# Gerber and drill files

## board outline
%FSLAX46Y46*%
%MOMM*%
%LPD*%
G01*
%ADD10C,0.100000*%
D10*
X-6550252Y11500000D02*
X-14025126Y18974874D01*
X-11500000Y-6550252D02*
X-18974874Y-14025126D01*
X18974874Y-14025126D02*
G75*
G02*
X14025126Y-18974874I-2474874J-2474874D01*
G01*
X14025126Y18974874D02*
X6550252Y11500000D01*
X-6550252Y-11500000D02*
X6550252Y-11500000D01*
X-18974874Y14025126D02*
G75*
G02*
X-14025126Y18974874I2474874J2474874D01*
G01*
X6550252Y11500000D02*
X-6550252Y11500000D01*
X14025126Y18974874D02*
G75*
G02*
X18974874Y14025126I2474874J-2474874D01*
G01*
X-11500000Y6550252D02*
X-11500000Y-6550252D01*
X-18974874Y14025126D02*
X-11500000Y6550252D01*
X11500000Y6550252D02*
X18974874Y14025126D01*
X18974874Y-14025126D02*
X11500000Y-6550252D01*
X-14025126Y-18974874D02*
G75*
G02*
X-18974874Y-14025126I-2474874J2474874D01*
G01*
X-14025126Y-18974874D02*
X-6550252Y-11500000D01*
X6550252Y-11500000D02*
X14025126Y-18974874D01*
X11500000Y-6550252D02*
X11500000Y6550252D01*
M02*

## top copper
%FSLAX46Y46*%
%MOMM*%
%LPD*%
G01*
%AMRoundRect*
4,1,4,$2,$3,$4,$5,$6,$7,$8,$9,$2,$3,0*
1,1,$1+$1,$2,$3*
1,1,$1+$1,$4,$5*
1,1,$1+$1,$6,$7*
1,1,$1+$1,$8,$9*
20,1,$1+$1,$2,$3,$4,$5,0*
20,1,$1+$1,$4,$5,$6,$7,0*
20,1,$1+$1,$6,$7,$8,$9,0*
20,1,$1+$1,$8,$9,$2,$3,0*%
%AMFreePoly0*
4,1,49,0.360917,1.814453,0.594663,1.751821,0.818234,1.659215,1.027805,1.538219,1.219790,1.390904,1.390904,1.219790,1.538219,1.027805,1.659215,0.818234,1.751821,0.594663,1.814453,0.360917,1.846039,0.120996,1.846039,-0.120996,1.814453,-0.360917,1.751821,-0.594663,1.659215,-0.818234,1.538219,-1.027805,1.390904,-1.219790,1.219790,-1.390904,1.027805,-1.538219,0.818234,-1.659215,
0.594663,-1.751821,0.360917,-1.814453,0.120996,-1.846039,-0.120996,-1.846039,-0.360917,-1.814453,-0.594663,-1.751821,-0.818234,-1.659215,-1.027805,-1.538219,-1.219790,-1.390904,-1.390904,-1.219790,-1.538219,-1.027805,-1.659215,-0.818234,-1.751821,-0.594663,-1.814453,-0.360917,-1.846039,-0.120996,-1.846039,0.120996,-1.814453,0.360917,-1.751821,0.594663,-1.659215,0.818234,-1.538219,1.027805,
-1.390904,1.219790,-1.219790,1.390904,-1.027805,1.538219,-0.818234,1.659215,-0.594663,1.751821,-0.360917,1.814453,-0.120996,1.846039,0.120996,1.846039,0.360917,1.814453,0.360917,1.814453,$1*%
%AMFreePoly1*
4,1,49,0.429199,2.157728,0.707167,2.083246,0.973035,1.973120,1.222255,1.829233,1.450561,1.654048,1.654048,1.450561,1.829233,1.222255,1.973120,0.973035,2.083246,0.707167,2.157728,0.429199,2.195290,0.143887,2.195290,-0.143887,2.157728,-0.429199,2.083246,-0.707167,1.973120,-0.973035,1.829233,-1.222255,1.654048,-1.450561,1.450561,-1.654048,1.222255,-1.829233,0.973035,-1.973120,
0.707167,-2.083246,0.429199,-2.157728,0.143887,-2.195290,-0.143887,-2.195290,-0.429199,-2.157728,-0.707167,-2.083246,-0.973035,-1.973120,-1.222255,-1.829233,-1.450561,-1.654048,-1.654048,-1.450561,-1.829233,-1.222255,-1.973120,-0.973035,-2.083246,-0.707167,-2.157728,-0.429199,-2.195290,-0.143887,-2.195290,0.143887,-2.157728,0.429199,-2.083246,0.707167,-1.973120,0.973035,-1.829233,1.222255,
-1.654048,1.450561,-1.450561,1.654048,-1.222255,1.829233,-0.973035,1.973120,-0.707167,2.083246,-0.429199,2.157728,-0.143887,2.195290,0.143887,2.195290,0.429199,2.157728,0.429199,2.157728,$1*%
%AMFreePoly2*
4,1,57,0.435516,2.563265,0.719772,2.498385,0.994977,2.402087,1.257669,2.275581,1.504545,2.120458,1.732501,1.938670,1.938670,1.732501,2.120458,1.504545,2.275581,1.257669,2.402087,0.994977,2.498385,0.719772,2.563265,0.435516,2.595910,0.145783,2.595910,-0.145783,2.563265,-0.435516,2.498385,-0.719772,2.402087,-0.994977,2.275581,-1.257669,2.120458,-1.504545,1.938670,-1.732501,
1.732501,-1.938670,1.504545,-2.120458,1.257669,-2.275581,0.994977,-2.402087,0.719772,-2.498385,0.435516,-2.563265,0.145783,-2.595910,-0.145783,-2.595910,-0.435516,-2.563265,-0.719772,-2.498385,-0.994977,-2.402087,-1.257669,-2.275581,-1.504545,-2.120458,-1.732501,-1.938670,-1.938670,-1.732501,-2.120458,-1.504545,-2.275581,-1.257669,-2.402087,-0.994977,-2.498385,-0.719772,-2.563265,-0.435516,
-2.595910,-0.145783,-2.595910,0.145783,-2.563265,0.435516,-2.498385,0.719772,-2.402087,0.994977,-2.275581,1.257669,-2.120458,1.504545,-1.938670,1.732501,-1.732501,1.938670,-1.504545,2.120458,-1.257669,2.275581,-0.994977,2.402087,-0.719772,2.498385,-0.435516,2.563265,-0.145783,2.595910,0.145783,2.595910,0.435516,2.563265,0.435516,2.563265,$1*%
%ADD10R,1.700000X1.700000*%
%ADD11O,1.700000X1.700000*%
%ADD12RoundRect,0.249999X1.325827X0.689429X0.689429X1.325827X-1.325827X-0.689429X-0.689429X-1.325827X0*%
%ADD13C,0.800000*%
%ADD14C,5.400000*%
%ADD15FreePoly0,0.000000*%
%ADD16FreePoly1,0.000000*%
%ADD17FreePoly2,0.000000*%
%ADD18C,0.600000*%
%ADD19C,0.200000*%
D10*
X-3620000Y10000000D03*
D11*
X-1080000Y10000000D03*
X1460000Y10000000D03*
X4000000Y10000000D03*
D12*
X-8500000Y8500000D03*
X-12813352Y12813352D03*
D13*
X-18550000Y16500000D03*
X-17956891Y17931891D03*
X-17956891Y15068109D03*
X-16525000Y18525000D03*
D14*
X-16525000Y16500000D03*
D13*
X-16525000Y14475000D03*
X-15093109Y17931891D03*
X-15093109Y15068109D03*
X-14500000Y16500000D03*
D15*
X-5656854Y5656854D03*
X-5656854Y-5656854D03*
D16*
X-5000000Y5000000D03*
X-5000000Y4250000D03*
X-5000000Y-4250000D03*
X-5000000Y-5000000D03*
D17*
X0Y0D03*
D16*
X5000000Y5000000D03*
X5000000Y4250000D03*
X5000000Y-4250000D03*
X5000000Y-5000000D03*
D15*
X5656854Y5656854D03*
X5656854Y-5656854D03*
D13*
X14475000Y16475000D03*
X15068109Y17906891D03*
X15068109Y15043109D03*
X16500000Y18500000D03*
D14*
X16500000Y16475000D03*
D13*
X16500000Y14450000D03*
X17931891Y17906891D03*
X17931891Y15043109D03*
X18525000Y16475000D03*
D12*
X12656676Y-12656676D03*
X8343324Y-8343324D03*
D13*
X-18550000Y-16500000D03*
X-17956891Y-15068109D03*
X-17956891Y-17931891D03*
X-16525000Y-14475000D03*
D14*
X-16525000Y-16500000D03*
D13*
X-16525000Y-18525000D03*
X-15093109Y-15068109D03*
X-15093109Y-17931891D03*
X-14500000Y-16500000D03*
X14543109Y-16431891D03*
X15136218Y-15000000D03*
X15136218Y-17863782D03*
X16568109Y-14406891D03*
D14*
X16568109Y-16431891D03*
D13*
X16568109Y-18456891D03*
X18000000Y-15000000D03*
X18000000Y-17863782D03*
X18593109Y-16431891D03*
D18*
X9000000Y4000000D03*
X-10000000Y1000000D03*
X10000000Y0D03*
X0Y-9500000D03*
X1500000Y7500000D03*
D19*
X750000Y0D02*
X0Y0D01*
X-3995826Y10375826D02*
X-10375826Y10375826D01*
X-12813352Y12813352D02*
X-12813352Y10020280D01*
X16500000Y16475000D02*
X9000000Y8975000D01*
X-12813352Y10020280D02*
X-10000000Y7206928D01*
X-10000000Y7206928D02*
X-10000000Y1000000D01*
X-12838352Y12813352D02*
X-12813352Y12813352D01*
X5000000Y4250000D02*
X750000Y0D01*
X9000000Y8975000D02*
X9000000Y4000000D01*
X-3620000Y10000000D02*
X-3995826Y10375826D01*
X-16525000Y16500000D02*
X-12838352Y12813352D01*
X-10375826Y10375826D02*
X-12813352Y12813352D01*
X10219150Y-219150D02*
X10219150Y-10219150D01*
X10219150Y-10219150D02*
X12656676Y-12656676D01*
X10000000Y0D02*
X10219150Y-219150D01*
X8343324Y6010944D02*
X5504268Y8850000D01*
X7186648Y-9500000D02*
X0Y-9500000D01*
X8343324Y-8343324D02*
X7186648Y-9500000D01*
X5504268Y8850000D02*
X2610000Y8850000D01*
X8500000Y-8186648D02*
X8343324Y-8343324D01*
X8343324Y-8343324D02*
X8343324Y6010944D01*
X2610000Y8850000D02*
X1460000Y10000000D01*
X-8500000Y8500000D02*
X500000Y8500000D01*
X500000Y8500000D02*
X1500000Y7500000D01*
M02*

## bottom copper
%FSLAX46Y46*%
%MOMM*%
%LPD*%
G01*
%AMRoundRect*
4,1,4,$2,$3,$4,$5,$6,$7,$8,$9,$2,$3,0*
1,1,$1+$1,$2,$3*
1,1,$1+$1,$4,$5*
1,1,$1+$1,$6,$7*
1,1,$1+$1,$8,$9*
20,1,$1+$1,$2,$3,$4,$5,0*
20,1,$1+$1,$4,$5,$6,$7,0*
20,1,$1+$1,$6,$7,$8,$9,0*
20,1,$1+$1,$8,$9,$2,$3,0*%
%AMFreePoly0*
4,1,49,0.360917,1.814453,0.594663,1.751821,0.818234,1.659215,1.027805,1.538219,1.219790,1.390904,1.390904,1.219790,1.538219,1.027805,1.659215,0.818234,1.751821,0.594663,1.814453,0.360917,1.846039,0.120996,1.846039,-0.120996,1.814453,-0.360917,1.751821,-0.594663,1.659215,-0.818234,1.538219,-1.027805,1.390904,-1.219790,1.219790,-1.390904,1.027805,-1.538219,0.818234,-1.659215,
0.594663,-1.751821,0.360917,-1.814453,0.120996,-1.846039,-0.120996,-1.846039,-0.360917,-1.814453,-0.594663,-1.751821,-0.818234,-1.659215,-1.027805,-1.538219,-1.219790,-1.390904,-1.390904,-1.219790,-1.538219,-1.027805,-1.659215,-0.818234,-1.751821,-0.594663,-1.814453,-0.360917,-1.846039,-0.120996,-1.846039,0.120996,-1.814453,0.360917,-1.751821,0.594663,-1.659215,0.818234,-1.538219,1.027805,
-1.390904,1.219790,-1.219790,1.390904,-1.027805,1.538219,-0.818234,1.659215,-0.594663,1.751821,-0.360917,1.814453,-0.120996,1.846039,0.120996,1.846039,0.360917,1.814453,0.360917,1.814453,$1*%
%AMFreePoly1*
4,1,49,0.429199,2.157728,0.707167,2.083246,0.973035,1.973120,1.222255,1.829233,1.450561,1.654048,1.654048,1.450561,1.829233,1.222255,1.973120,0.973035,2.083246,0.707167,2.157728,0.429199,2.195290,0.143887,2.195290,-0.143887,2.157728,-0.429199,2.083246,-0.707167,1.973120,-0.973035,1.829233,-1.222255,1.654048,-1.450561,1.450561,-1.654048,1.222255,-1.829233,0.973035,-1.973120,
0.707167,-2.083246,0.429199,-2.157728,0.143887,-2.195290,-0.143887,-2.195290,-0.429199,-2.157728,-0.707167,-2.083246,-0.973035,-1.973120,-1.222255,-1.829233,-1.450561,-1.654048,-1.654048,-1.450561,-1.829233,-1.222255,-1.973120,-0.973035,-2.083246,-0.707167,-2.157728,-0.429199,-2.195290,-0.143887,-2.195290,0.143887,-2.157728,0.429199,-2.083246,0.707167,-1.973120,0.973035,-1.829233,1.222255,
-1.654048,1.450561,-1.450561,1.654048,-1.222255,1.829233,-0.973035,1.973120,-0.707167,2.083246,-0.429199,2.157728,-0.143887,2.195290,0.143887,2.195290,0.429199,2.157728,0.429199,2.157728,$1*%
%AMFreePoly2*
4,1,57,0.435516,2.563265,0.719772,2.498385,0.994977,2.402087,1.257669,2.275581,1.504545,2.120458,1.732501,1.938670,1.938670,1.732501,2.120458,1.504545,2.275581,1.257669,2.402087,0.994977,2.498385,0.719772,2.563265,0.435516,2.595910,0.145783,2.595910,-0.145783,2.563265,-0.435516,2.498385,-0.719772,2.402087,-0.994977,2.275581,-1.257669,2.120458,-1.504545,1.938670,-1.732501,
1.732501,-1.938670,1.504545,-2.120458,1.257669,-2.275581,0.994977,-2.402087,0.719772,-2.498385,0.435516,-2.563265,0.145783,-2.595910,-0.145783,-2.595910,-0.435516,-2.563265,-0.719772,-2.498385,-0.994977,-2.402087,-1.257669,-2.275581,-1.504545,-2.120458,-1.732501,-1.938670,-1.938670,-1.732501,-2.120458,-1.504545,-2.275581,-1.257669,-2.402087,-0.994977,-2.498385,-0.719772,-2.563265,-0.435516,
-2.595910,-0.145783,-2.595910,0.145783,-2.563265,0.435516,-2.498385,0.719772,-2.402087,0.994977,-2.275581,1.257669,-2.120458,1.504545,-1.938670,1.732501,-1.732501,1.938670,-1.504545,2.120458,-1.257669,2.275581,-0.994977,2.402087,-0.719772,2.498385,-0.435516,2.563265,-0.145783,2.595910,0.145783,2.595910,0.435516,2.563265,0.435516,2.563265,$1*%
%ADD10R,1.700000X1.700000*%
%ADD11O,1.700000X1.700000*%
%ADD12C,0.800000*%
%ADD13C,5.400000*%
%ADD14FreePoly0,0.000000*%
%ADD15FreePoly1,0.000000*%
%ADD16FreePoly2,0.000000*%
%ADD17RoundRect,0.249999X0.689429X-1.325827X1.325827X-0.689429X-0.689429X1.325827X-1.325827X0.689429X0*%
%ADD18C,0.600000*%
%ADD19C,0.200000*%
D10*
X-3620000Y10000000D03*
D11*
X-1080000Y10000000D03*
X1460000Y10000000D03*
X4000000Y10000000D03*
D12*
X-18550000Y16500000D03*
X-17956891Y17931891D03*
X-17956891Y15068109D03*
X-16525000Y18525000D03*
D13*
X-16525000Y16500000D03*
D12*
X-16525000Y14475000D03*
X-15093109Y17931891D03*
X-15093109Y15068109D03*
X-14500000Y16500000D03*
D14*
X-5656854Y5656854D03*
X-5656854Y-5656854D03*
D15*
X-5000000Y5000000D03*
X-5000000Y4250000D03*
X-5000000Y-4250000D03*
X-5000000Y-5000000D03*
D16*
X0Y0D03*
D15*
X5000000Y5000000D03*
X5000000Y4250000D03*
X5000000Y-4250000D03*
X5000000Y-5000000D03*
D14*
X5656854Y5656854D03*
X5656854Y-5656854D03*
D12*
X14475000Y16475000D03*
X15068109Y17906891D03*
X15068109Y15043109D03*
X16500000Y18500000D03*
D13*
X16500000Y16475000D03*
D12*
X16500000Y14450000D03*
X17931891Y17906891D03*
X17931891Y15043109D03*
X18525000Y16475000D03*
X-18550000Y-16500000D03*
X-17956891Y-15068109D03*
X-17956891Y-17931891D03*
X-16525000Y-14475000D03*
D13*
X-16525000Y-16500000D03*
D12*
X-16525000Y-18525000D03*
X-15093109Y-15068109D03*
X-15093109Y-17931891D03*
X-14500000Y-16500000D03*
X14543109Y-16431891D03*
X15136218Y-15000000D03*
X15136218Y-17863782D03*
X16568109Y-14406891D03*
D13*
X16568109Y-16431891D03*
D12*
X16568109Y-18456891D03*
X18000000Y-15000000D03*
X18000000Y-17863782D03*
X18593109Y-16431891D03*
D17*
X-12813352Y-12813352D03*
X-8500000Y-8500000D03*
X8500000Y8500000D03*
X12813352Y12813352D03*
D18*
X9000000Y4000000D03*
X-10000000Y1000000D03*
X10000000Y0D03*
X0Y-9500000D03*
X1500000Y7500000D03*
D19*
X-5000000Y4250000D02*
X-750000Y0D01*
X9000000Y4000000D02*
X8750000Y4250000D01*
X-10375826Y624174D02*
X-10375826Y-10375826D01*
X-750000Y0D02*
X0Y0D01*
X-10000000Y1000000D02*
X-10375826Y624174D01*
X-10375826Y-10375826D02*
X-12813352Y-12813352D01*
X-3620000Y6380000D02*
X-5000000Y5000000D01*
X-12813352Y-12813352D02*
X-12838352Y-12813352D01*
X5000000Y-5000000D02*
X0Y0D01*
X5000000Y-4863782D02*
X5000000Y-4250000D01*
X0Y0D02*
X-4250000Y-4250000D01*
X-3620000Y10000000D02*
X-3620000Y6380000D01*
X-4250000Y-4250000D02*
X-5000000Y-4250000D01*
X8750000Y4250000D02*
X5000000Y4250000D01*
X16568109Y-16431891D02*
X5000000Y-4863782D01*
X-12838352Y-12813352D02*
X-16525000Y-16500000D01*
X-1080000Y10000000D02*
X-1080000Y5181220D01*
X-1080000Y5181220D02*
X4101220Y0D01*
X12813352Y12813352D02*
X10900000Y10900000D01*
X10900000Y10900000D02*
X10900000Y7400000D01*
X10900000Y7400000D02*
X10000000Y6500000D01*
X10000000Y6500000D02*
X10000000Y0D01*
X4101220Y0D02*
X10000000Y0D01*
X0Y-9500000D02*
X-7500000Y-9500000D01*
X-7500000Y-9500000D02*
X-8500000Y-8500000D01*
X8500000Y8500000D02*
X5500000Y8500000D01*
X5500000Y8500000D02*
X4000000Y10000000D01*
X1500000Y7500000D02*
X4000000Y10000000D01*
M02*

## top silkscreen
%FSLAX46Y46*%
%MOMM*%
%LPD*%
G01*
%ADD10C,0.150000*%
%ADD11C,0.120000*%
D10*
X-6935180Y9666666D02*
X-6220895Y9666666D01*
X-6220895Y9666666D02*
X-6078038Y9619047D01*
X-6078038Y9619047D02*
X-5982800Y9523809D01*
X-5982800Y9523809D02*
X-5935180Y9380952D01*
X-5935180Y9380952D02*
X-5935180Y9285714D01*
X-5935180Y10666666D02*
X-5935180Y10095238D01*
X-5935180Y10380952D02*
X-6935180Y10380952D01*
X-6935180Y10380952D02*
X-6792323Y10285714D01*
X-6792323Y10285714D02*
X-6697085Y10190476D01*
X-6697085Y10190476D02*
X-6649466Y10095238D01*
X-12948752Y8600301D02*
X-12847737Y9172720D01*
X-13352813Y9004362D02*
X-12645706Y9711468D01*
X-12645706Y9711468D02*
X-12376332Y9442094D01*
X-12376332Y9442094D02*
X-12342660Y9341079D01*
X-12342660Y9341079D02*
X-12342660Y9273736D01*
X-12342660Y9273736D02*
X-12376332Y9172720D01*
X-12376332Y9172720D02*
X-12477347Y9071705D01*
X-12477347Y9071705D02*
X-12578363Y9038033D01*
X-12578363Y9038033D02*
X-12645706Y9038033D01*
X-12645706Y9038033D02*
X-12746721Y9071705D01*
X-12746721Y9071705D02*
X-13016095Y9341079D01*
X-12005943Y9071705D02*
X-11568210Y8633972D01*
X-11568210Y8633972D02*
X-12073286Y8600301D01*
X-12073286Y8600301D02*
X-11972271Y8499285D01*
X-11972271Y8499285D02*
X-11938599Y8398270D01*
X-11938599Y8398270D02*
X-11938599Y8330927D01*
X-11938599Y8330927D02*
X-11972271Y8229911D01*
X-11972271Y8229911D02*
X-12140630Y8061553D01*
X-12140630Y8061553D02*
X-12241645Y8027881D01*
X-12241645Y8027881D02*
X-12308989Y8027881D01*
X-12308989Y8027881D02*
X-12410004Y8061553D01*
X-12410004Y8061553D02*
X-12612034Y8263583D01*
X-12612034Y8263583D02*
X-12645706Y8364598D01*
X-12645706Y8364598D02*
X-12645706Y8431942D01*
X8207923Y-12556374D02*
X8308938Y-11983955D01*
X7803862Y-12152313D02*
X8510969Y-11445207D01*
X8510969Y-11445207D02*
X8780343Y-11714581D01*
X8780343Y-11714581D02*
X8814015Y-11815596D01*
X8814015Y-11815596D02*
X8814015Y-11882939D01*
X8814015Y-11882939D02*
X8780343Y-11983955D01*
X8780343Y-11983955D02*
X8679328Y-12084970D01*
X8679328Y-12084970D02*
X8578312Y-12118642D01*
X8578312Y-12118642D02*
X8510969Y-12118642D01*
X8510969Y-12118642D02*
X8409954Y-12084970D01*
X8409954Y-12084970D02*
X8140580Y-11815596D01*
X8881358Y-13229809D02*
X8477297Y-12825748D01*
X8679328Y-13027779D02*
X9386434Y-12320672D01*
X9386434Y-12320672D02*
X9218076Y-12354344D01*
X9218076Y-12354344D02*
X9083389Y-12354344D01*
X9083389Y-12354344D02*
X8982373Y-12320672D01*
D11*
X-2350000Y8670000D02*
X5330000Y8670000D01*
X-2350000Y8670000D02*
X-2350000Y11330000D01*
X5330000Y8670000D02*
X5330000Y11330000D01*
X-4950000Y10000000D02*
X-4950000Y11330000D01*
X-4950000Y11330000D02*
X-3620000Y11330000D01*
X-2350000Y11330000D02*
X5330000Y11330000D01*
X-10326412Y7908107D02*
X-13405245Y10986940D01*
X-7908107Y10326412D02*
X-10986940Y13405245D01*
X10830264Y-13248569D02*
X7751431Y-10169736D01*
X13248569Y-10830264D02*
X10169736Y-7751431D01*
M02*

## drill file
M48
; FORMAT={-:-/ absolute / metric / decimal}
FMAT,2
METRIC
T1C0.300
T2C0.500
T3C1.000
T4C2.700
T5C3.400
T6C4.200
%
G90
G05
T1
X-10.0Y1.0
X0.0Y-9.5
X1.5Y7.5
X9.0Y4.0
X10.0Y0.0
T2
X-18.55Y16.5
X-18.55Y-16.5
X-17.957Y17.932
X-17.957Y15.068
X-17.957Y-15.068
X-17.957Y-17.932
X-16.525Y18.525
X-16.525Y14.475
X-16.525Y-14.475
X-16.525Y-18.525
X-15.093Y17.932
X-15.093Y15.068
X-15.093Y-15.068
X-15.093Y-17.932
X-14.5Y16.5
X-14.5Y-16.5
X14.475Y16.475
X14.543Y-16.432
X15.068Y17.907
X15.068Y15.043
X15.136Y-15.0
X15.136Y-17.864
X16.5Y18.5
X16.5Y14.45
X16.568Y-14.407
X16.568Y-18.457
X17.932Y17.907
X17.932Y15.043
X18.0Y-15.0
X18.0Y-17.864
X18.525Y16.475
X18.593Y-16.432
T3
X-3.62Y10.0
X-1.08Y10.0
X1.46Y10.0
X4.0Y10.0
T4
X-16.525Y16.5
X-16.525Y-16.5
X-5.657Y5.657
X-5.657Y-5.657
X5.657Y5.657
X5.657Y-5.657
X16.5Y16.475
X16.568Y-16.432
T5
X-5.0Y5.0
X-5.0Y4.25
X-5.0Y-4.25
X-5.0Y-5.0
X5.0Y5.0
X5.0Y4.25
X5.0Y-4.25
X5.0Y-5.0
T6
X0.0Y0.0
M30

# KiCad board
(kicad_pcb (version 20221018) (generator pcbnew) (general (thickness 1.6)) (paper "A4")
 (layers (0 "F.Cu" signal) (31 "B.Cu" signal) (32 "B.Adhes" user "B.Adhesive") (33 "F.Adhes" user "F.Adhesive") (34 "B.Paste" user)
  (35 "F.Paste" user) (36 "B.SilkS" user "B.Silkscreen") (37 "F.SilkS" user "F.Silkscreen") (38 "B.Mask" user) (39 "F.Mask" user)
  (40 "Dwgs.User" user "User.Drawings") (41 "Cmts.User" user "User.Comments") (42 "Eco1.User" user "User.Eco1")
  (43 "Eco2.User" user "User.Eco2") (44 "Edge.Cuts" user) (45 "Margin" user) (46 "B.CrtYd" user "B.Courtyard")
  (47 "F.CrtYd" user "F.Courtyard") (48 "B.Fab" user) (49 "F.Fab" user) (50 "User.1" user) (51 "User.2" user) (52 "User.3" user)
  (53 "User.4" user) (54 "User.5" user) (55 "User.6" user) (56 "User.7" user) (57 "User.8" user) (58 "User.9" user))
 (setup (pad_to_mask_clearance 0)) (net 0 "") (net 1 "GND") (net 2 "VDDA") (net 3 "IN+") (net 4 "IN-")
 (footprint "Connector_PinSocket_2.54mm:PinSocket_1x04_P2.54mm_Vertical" (layer "F.Cu") (at -3.62 -10 90)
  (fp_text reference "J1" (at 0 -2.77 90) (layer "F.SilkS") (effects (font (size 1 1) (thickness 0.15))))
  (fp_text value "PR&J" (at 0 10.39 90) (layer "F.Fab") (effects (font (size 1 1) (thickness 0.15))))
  (fp_line (start -1.33 1.27) (end -1.33 8.95) (stroke (width 0.12) (type solid)) (layer "F.SilkS"))
  (fp_line (start -1.33 1.27) (end 1.33 1.27) (stroke (width 0.12) (type solid)) (layer "F.SilkS"))
  (fp_line (start -1.33 8.95) (end 1.33 8.95) (stroke (width 0.12) (type solid)) (layer "F.SilkS"))
  (fp_line (start 0 -1.33) (end 1.33 -1.33) (stroke (width 0.12) (type solid)) (layer "F.SilkS"))
  (fp_line (start 1.33 -1.33) (end 1.33 0) (stroke (width 0.12) (type solid)) (layer "F.SilkS"))
  (fp_line (start 1.33 1.27) (end 1.33 8.95) (stroke (width 0.12) (type solid)) (layer "F.SilkS"))
  (pad "1" thru_hole rect (at 0 0 90) (size 1.7 1.7) (drill 1) (layers "*.Cu" "*.Mask") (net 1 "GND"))
  (pad "2" thru_hole oval (at 0 2.54 90) (size 1.7 1.7) (drill 1) (layers "*.Cu" "*.Mask") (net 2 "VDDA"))
  (pad "3" thru_hole oval (at 0 5.08 90) (size 1.7 1.7) (drill 1) (layers "*.Cu" "*.Mask") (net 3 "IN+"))
  (pad "4" thru_hole oval (at 0 7.62 90) (size 1.7 1.7) (drill 1) (layers "*.Cu" "*.Mask") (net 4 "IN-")))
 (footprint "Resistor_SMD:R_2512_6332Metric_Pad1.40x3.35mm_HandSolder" (layer "F.Cu") (at -10.656676 -10.656676 135)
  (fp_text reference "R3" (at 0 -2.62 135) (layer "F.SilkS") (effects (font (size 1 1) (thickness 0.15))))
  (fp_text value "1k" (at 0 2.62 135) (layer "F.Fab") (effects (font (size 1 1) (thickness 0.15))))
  (fp_line (start -2.177064 -1.71) (end 2.177064 -1.71) (stroke (width 0.12) (type solid)) (layer "F.SilkS"))
  (fp_line (start -2.177064 1.71) (end 2.177064 1.71) (stroke (width 0.12) (type solid)) (layer "F.SilkS"))
  (pad "1" smd roundrect (at -3.05 0 135) (size 1.4 3.35) (layers "F.Cu" "F.Paste" "F.Mask") (roundrect_rratio 0.1785707143) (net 4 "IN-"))
  (pad "2" smd roundrect (at 3.05 0 135) (size 1.4 3.35) (layers "F.Cu" "F.Paste" "F.Mask") (roundrect_rratio 0.1785707143) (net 1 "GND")))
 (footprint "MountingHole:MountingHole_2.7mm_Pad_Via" (layer "F.Cu") (at -16.525 -16.5)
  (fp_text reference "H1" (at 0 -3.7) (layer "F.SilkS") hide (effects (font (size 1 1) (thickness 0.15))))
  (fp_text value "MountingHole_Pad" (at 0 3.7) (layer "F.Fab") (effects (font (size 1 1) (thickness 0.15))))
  (pad "1" thru_hole circle (at -2.025 0) (size 0.8 0.8) (drill 0.5) (layers "*.Cu" "*.Mask") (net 1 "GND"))
  (pad "1" thru_hole circle (at -1.431891 -1.431891) (size 0.8 0.8) (drill 0.5) (layers "*.Cu" "*.Mask") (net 1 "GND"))
  (pad "1" thru_hole circle (at -1.431891 1.431891) (size 0.8 0.8) (drill 0.5) (layers "*.Cu" "*.Mask") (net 1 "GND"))
  (pad "1" thru_hole circle (at 0 -2.025) (size 0.8 0.8) (drill 0.5) (layers "*.Cu" "*.Mask") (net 1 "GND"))
  (pad "1" thru_hole circle (at 0 0) (size 5.4 5.4) (drill 2.7) (layers "*.Cu" "*.Mask") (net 1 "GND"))
  (pad "1" thru_hole circle (at 0 2.025) (size 0.8 0.8) (drill 0.5) (layers "*.Cu" "*.Mask") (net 1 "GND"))
  (pad "1" thru_hole circle (at 1.431891 -1.431891) (size 0.8 0.8) (drill 0.5) (layers "*.Cu" "*.Mask") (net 1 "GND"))
  (pad "1" thru_hole circle (at 1.431891 1.431891) (size 0.8 0.8) (drill 0.5) (layers "*.Cu" "*.Mask") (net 1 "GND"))
  (pad "1" thru_hole circle (at 2.025 0) (size 0.8 0.8) (drill 0.5) (layers "*.Cu" "*.Mask") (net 1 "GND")))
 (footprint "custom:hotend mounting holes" (layer "F.Cu") (at 0 0)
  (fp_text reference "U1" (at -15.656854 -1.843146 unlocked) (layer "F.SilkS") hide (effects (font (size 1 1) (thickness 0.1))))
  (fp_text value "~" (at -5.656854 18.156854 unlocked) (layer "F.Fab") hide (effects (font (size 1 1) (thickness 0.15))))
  (pad "1" thru_hole custom (at -5.656854 -5.656854) (size 3.7 3.7) (drill 2.7) (layers "*.Cu" "*.Mask") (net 1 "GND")
   (thermal_bridge_angle 45) (options (clearance outline) (anchor circle)) (primitives))
  (pad "1" thru_hole custom (at -5.656854 5.656854) (size 3.7 3.7) (drill 2.7) (layers "*.Cu" "*.Mask") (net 1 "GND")
   (thermal_bridge_angle 45) (options (clearance outline) (anchor circle)) (primitives))
  (pad "1" thru_hole custom (at -5 -5) (size 4.4 4.4) (drill 3.4) (layers "*.Cu" "*.Mask") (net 1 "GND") (thermal_bridge_angle 45)
   (options (clearance outline) (anchor circle)) (primitives))
  (pad "1" thru_hole custom (at -5 -4.25) (size 4.4 4.4) (drill 3.4) (layers "*.Cu" "*.Mask") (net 1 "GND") (thermal_bridge_angle 45)
   (options (clearance outline) (anchor circle)) (primitives))
  (pad "1" thru_hole custom (at -5 4.25) (size 4.4 4.4) (drill 3.4) (layers "*.Cu" "*.Mask") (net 1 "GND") (thermal_bridge_angle 45)
   (options (clearance outline) (anchor circle)) (primitives))
  (pad "1" thru_hole custom (at -5 5) (size 4.4 4.4) (drill 3.4) (layers "*.Cu" "*.Mask") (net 1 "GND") (thermal_bridge_angle 45)
   (options (clearance outline) (anchor circle)) (primitives))
  (pad "1" thru_hole custom (at 0 0) (size 5.2 5.2) (drill 4.2) (layers "*.Cu" "*.Mask") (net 1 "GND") (thermal_bridge_angle 45)
   (options (clearance outline) (anchor circle)) (primitives))
  (pad "1" thru_hole custom (at 5 -5) (size 4.4 4.4) (drill 3.4) (layers "*.Cu" "*.Mask") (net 1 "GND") (thermal_bridge_angle 45)
   (options (clearance outline) (anchor circle)) (primitives))
  (pad "1" thru_hole custom (at 5 -4.25) (size 4.4 4.4) (drill 3.4) (layers "*.Cu" "*.Mask") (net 1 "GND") (thermal_bridge_angle 45)
   (options (clearance outline) (anchor circle)) (primitives))
  (pad "1" thru_hole custom (at 5 4.25) (size 4.4 4.4) (drill 3.4) (layers "*.Cu" "*.Mask") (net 1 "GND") (thermal_bridge_angle 45)
   (options (clearance outline) (anchor circle)) (primitives))
  (pad "1" thru_hole custom (at 5 5) (size 4.4 4.4) (drill 3.4) (layers "*.Cu" "*.Mask") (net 1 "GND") (thermal_bridge_angle 45)
   (options (clearance outline) (anchor circle)) (primitives))
  (pad "1" thru_hole custom (at 5.656854 -5.656854) (size 3.7 3.7) (drill 2.7) (layers "*.Cu" "*.Mask") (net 1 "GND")
   (thermal_bridge_angle 45) (options (clearance outline) (anchor circle)) (primitives))
  (pad "1" thru_hole custom (at 5.656854 5.656854) (size 3.7 3.7) (drill 2.7) (layers "*.Cu" "*.Mask") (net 1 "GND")
   (thermal_bridge_angle 45) (options (clearance outline) (anchor circle)) (primitives)))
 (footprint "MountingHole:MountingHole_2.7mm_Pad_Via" (layer "F.Cu") (at 16.5 -16.475)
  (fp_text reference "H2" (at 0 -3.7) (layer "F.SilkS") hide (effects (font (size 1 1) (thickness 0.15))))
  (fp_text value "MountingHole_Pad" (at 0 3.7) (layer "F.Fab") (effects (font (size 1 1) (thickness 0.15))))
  (pad "1" thru_hole circle (at -2.025 0) (size 0.8 0.8) (drill 0.5) (layers "*.Cu" "*.Mask") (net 1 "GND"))
  (pad "1" thru_hole circle (at -1.431891 -1.431891) (size 0.8 0.8) (drill 0.5) (layers "*.Cu" "*.Mask") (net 1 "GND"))
  (pad "1" thru_hole circle (at -1.431891 1.431891) (size 0.8 0.8) (drill 0.5) (layers "*.Cu" "*.Mask") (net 1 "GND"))
  (pad "1" thru_hole circle (at 0 -2.025) (size 0.8 0.8) (drill 0.5) (layers "*.Cu" "*.Mask") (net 1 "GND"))
  (pad "1" thru_hole circle (at 0 0) (size 5.4 5.4) (drill 2.7) (layers "*.Cu" "*.Mask") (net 1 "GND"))
  (pad "1" thru_hole circle (at 0 2.025) (size 0.8 0.8) (drill 0.5) (layers "*.Cu" "*.Mask") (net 1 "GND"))
  (pad "1" thru_hole circle (at 1.431891 -1.431891) (size 0.8 0.8) (drill 0.5) (layers "*.Cu" "*.Mask") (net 1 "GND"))
  (pad "1" thru_hole circle (at 1.431891 1.431891) (size 0.8 0.8) (drill 0.5) (layers "*.Cu" "*.Mask") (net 1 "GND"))
  (pad "1" thru_hole circle (at 2.025 0) (size 0.8 0.8) (drill 0.5) (layers "*.Cu" "*.Mask") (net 1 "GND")))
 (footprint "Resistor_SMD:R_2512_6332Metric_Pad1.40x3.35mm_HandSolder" (layer "F.Cu") (at 10.5 10.5 135)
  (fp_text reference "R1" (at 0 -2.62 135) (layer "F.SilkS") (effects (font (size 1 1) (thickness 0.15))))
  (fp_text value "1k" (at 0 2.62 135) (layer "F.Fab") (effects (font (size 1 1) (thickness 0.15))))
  (fp_line (start -2.177064 -1.71) (end 2.177064 -1.71) (stroke (width 0.12) (type solid)) (layer "F.SilkS"))
  (fp_line (start -2.177064 1.71) (end 2.177064 1.71) (stroke (width 0.12) (type solid)) (layer "F.SilkS"))
  (pad "1" smd roundrect (at -3.05 0 135) (size 1.4 3.35) (layers "F.Cu" "F.Paste" "F.Mask") (roundrect_rratio 0.1785707143) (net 2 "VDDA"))
  (pad "2" smd roundrect (at 3.05 0 135) (size 1.4 3.35) (layers "F.Cu" "F.Paste" "F.Mask") (roundrect_rratio 0.1785707143) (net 3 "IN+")))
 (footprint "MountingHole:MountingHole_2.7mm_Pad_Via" (layer "F.Cu") (at -16.525 16.5)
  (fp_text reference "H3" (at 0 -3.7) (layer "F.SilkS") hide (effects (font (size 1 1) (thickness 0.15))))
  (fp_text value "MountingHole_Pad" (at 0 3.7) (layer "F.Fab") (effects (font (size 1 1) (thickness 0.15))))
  (pad "1" thru_hole circle (at -2.025 0) (size 0.8 0.8) (drill 0.5) (layers "*.Cu" "*.Mask") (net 1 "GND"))
  (pad "1" thru_hole circle (at -1.431891 -1.431891) (size 0.8 0.8) (drill 0.5) (layers "*.Cu" "*.Mask") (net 1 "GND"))
  (pad "1" thru_hole circle (at -1.431891 1.431891) (size 0.8 0.8) (drill 0.5) (layers "*.Cu" "*.Mask") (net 1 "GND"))
  (pad "1" thru_hole circle (at 0 -2.025) (size 0.8 0.8) (drill 0.5) (layers "*.Cu" "*.Mask") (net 1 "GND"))
  (pad "1" thru_hole circle (at 0 0) (size 5.4 5.4) (drill 2.7) (layers "*.Cu" "*.Mask") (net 1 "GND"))
  (pad "1" thru_hole circle (at 0 2.025) (size 0.8 0.8) (drill 0.5) (layers "*.Cu" "*.Mask") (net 1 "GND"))
  (pad "1" thru_hole circle (at 1.431891 -1.431891) (size 0.8 0.8) (drill 0.5) (layers "*.Cu" "*.Mask") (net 1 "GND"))
  (pad "1" thru_hole circle (at 1.431891 1.431891) (size 0.8 0.8) (drill 0.5) (layers "*.Cu" "*.Mask") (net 1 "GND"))
  (pad "1" thru_hole circle (at 2.025 0) (size 0.8 0.8) (drill 0.5) (layers "*.Cu" "*.Mask") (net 1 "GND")))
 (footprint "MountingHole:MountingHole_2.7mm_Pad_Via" (layer "F.Cu") (at 16.568109 16.431891)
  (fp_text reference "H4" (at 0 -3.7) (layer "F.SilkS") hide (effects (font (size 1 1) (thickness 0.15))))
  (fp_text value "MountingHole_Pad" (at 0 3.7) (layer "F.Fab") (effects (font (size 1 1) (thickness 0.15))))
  (pad "1" thru_hole circle (at -2.025 0) (size 0.8 0.8) (drill 0.5) (layers "*.Cu" "*.Mask") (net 1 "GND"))
  (pad "1" thru_hole circle (at -1.431891 -1.431891) (size 0.8 0.8) (drill 0.5) (layers "*.Cu" "*.Mask") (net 1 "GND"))
  (pad "1" thru_hole circle (at -1.431891 1.431891) (size 0.8 0.8) (drill 0.5) (layers "*.Cu" "*.Mask") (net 1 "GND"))
  (pad "1" thru_hole circle (at 0 -2.025) (size 0.8 0.8) (drill 0.5) (layers "*.Cu" "*.Mask") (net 1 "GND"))
  (pad "1" thru_hole circle (at 0 0) (size 5.4 5.4) (drill 2.7) (layers "*.Cu" "*.Mask") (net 1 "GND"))
  (pad "1" thru_hole circle (at 0 2.025) (size 0.8 0.8) (drill 0.5) (layers "*.Cu" "*.Mask") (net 1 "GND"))
  (pad "1" thru_hole circle (at 1.431891 -1.431891) (size 0.8 0.8) (drill 0.5) (layers "*.Cu" "*.Mask") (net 1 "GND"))
  (pad "1" thru_hole circle (at 1.431891 1.431891) (size 0.8 0.8) (drill 0.5) (layers "*.Cu" "*.Mask") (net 1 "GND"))
  (pad "1" thru_hole circle (at 2.025 0) (size 0.8 0.8) (drill 0.5) (layers "*.Cu" "*.Mask") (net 1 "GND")))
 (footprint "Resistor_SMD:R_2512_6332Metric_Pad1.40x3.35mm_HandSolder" (layer "B.Cu") (at -10.656676 10.656676 45)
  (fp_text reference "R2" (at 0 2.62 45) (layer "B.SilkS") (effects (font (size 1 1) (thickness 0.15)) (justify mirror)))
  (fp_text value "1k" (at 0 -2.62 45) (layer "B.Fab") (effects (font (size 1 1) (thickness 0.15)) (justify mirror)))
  (pad "1" smd roundrect (at -3.05 0 45) (size 1.4 3.35) (layers "B.Cu" "B.Paste" "B.Mask") (roundrect_rratio 0.1785707143) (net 1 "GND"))
  (pad "2" smd roundrect (at 3.05 0 45) (size 1.4 3.35) (layers "B.Cu" "B.Paste" "B.Mask") (roundrect_rratio 0.1785707143) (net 3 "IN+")))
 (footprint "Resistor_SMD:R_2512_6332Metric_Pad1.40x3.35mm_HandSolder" (layer "B.Cu") (at 10.656676 -10.656676 45)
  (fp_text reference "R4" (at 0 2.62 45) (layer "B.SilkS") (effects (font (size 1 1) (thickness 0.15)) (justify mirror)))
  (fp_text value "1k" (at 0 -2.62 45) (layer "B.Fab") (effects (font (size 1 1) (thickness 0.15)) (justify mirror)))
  (pad "1" smd roundrect (at -3.05 0 45) (size 1.4 3.35) (layers "B.Cu" "B.Paste" "B.Mask") (roundrect_rratio 0.1785707143) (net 4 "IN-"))
  (pad "2" smd roundrect (at 3.05 0 45) (size 1.4 3.35) (layers "B.Cu" "B.Paste" "B.Mask") (roundrect_rratio 0.1785707143) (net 2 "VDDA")))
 (gr_line (start -6.550252 -11.5) (end -14.025126 -18.974874) (stroke (width 0.1) (type solid)) (layer "Edge.Cuts"))
 (gr_line (start -11.5 6.550252) (end -18.974874 14.025126) (stroke (width 0.1) (type solid)) (layer "Edge.Cuts"))
 (gr_arc (start 18.974874 14.025126) (mid 18.974874 18.974874) (end 14.025126 18.974874) (stroke (width 0.1) (type solid))
  (layer "Edge.Cuts"))
 (gr_line (start 14.025126 -18.974874) (end 6.550252 -11.5) (stroke (width 0.1) (type solid)) (layer "Edge.Cuts"))
 (gr_line (start -6.550252 11.5) (end 6.550252 11.5) (stroke (width 0.1) (type solid)) (layer "Edge.Cuts"))
 (gr_arc (start -18.974874 -14.025126) (mid -18.974874 -18.974874) (end -14.025126 -18.974874) (stroke (width 0.1) (type solid))
  (layer "Edge.Cuts"))
 (gr_line (start 6.550252 -11.5) (end -6.550252 -11.5) (stroke (width 0.1) (type solid)) (layer "Edge.Cuts"))
 (gr_arc (start 14.025126 -18.974874) (mid 18.974874 -18.974874) (end 18.974874 -14.025126) (stroke (width 0.1) (type solid))
  (layer "Edge.Cuts"))
 (gr_line (start -11.5 -6.550252) (end -11.5 6.550252) (stroke (width 0.1) (type solid)) (layer "Edge.Cuts"))
 (gr_line (start -18.974874 -14.025126) (end -11.5 -6.550252) (stroke (width 0.1) (type solid)) (layer "Edge.Cuts"))
 (gr_line (start 11.5 -6.550252) (end 18.974874 -14.025126) (stroke (width 0.1) (type solid)) (layer "Edge.Cuts"))
 (gr_line (start 18.974874 14.025126) (end 11.5 6.550252) (stroke (width 0.1) (type solid)) (layer "Edge.Cuts"))
 (gr_arc (start -14.025126 18.974874) (mid -18.974874 18.974874) (end -18.974874 14.025126) (stroke (width 0.1) (type solid))
  (layer "Edge.Cuts"))
 (gr_line (start -14.025126 18.974874) (end -6.550252 11.5) (stroke (width 0.1) (type solid)) (layer "Edge.Cuts"))
 (gr_line (start 6.550252 11.5) (end 14.025126 18.974874) (stroke (width 0.1) (type solid)) (layer "Edge.Cuts"))
 (gr_line (start 11.5 6.550252) (end 11.5 -6.550252) (stroke (width 0.1) (type solid)) (layer "Edge.Cuts"))
 (segment (start 0.75 0) (end 0 0) (width 0.2) (layer "F.Cu") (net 1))
 (segment (start -3.995826 -10.375826) (end -10.375826 -10.375826) (width 0.2) (layer "F.Cu") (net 1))
 (segment (start -12.813352 -12.813352) (end -12.813352 -10.02028) (width 0.2) (layer "F.Cu") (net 1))
 (segment (start 16.5 -16.475) (end 9 -8.975) (width 0.2) (layer "F.Cu") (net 1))
 (segment (start -12.813352 -10.02028) (end -10 -7.206928) (width 0.2) (layer "F.Cu") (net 1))
 (segment (start -10 -7.206928) (end -10 -1) (width 0.2) (layer "F.Cu") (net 1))
 (segment (start -12.838352 -12.813352) (end -12.813352 -12.813352) (width 0.2) (layer "F.Cu") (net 1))
 (segment (start 5 -4.25) (end 0.75 0) (width 0.2) (layer "F.Cu") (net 1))
 (segment (start 9 -8.975) (end 9 -4) (width 0.2) (layer "F.Cu") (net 1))
 (segment (start -3.62 -10) (end -3.995826 -10.375826) (width 0.2) (layer "F.Cu") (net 1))
 (segment (start -16.525 -16.5) (end -12.838352 -12.813352) (width 0.2) (layer "F.Cu") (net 1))
 (segment (start -10.375826 -10.375826) (end -12.813352 -12.813352) (width 0.2) (layer "F.Cu") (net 1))
 (via (at 9 -4) (size 0.6) (drill 0.3) (layers "F.Cu" "B.Cu") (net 1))
 (via (at -10 -1) (size 0.6) (drill 0.3) (layers "F.Cu" "B.Cu") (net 1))
 (segment (start -5 -4.25) (end -0.75 0) (width 0.2) (layer "B.Cu") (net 1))
 (segment (start 9 -4) (end 8.75 -4.25) (width 0.2) (layer "B.Cu") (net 1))
 (segment (start -10.375826 -0.624174) (end -10.375826 10.375826) (width 0.2) (layer "B.Cu") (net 1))
 (segment (start -0.75 0) (end 0 0) (width 0.2) (layer "B.Cu") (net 1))
 (segment (start -10 -1) (end -10.375826 -0.624174) (width 0.2) (layer "B.Cu") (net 1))
 (segment (start -10.375826 10.375826) (end -12.813352 12.813352) (width 0.2) (layer "B.Cu") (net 1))
 (segment (start -3.62 -6.38) (end -5 -5) (width 0.2) (layer "B.Cu") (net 1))
 (segment (start -12.813352 12.813352) (end -12.838352 12.813352) (width 0.2) (layer "B.Cu") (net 1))
 (segment (start 5 5) (end 0 0) (width 0.2) (layer "B.Cu") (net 1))
 (segment (start 5 4.863782) (end 5 4.25) (width 0.2) (layer "B.Cu") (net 1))
 (segment (start 0 0) (end -4.25 4.25) (width 0.2) (layer "B.Cu") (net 1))
 (segment (start -3.62 -10) (end -3.62 -6.38) (width 0.2) (layer "B.Cu") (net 1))
 (segment (start -4.25 4.25) (end -5 4.25) (width 0.2) (layer "B.Cu") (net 1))
 (segment (start 8.75 -4.25) (end 5 -4.25) (width 0.2) (layer "B.Cu") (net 1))
 (segment (start 16.568109 16.431891) (end 5 4.863782) (width 0.2) (layer "B.Cu") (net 1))
 (segment (start -12.838352 12.813352) (end -16.525 16.5) (width 0.2) (layer "B.Cu") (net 1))
 (segment (start 10.21915 0.21915) (end 10.21915 10.21915) (width 0.2) (layer "F.Cu") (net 2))
 (segment (start 10.21915 10.21915) (end 12.656676 12.656676) (width 0.2) (layer "F.Cu") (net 2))
 (segment (start 10 0) (end 10.21915 0.21915) (width 0.2) (layer "F.Cu") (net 2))
 (via (at 10 0) (size 0.6) (drill 0.3) (layers "F.Cu" "B.Cu") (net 2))
 (segment (start -1.08 -10) (end -1.08 -5.18122) (width 0.2) (layer "B.Cu") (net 2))
 (segment (start -1.08 -5.18122) (end 4.10122 0) (width 0.2) (layer "B.Cu") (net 2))
 (segment (start 12.813352 -12.813352) (end 10.9 -10.9) (width 0.2) (layer "B.Cu") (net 2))
 (segment (start 10.9 -10.9) (end 10.9 -7.4) (width 0.2) (layer "B.Cu") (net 2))
 (segment (start 10.9 -7.4) (end 10 -6.5) (width 0.2) (layer "B.Cu") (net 2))
 (segment (start 10 -6.5) (end 10 0) (width 0.2) (layer "B.Cu") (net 2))
 (segment (start 4.10122 0) (end 10 0) (width 0.2) (layer "B.Cu") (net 2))
 (segment (start 8.343324 -6.010944) (end 5.504268 -8.85) (width 0.2) (layer "F.Cu") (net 3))
 (segment (start 7.186648 9.5) (end 0 9.5) (width 0.2) (layer "F.Cu") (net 3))
 (segment (start 8.343324 8.343324) (end 7.186648 9.5) (width 0.2) (layer "F.Cu") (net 3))
 (segment (start 5.504268 -8.85) (end 2.61 -8.85) (width 0.2) (layer "F.Cu") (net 3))
 (segment (start 8.5 8.186648) (end 8.343324 8.343324) (width 0.2) (layer "F.Cu") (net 3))
 (segment (start 8.343324 8.343324) (end 8.343324 -6.010944) (width 0.2) (layer "F.Cu") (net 3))
 (segment (start 2.61 -8.85) (end 1.46 -10) (width 0.2) (layer "F.Cu") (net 3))
 (via (at 0 9.5) (size 0.6) (drill 0.3) (layers "F.Cu" "B.Cu") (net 3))
 (segment (start 0 9.5) (end -7.5 9.5) (width 0.2) (layer "B.Cu") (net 3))
 (segment (start -7.5 9.5) (end -8.5 8.5) (width 0.2) (layer "B.Cu") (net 3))
 (segment (start -8.5 -8.5) (end 0.5 -8.5) (width 0.2) (layer "F.Cu") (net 4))
 (segment (start 0.5 -8.5) (end 1.5 -7.5) (width 0.2) (layer "F.Cu") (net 4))
 (via (at 1.5 -7.5) (size 0.6) (drill 0.3) (layers "F.Cu" "B.Cu") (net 4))
 (segment (start 8.5 -8.5) (end 5.5 -8.5) (width 0.2) (layer "B.Cu") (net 4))
 (segment (start 5.5 -8.5) (end 4 -10) (width 0.2) (layer "B.Cu") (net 4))
 (segment (start 1.5 -7.5) (end 4 -10) (width 0.2) (layer "B.Cu") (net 4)))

